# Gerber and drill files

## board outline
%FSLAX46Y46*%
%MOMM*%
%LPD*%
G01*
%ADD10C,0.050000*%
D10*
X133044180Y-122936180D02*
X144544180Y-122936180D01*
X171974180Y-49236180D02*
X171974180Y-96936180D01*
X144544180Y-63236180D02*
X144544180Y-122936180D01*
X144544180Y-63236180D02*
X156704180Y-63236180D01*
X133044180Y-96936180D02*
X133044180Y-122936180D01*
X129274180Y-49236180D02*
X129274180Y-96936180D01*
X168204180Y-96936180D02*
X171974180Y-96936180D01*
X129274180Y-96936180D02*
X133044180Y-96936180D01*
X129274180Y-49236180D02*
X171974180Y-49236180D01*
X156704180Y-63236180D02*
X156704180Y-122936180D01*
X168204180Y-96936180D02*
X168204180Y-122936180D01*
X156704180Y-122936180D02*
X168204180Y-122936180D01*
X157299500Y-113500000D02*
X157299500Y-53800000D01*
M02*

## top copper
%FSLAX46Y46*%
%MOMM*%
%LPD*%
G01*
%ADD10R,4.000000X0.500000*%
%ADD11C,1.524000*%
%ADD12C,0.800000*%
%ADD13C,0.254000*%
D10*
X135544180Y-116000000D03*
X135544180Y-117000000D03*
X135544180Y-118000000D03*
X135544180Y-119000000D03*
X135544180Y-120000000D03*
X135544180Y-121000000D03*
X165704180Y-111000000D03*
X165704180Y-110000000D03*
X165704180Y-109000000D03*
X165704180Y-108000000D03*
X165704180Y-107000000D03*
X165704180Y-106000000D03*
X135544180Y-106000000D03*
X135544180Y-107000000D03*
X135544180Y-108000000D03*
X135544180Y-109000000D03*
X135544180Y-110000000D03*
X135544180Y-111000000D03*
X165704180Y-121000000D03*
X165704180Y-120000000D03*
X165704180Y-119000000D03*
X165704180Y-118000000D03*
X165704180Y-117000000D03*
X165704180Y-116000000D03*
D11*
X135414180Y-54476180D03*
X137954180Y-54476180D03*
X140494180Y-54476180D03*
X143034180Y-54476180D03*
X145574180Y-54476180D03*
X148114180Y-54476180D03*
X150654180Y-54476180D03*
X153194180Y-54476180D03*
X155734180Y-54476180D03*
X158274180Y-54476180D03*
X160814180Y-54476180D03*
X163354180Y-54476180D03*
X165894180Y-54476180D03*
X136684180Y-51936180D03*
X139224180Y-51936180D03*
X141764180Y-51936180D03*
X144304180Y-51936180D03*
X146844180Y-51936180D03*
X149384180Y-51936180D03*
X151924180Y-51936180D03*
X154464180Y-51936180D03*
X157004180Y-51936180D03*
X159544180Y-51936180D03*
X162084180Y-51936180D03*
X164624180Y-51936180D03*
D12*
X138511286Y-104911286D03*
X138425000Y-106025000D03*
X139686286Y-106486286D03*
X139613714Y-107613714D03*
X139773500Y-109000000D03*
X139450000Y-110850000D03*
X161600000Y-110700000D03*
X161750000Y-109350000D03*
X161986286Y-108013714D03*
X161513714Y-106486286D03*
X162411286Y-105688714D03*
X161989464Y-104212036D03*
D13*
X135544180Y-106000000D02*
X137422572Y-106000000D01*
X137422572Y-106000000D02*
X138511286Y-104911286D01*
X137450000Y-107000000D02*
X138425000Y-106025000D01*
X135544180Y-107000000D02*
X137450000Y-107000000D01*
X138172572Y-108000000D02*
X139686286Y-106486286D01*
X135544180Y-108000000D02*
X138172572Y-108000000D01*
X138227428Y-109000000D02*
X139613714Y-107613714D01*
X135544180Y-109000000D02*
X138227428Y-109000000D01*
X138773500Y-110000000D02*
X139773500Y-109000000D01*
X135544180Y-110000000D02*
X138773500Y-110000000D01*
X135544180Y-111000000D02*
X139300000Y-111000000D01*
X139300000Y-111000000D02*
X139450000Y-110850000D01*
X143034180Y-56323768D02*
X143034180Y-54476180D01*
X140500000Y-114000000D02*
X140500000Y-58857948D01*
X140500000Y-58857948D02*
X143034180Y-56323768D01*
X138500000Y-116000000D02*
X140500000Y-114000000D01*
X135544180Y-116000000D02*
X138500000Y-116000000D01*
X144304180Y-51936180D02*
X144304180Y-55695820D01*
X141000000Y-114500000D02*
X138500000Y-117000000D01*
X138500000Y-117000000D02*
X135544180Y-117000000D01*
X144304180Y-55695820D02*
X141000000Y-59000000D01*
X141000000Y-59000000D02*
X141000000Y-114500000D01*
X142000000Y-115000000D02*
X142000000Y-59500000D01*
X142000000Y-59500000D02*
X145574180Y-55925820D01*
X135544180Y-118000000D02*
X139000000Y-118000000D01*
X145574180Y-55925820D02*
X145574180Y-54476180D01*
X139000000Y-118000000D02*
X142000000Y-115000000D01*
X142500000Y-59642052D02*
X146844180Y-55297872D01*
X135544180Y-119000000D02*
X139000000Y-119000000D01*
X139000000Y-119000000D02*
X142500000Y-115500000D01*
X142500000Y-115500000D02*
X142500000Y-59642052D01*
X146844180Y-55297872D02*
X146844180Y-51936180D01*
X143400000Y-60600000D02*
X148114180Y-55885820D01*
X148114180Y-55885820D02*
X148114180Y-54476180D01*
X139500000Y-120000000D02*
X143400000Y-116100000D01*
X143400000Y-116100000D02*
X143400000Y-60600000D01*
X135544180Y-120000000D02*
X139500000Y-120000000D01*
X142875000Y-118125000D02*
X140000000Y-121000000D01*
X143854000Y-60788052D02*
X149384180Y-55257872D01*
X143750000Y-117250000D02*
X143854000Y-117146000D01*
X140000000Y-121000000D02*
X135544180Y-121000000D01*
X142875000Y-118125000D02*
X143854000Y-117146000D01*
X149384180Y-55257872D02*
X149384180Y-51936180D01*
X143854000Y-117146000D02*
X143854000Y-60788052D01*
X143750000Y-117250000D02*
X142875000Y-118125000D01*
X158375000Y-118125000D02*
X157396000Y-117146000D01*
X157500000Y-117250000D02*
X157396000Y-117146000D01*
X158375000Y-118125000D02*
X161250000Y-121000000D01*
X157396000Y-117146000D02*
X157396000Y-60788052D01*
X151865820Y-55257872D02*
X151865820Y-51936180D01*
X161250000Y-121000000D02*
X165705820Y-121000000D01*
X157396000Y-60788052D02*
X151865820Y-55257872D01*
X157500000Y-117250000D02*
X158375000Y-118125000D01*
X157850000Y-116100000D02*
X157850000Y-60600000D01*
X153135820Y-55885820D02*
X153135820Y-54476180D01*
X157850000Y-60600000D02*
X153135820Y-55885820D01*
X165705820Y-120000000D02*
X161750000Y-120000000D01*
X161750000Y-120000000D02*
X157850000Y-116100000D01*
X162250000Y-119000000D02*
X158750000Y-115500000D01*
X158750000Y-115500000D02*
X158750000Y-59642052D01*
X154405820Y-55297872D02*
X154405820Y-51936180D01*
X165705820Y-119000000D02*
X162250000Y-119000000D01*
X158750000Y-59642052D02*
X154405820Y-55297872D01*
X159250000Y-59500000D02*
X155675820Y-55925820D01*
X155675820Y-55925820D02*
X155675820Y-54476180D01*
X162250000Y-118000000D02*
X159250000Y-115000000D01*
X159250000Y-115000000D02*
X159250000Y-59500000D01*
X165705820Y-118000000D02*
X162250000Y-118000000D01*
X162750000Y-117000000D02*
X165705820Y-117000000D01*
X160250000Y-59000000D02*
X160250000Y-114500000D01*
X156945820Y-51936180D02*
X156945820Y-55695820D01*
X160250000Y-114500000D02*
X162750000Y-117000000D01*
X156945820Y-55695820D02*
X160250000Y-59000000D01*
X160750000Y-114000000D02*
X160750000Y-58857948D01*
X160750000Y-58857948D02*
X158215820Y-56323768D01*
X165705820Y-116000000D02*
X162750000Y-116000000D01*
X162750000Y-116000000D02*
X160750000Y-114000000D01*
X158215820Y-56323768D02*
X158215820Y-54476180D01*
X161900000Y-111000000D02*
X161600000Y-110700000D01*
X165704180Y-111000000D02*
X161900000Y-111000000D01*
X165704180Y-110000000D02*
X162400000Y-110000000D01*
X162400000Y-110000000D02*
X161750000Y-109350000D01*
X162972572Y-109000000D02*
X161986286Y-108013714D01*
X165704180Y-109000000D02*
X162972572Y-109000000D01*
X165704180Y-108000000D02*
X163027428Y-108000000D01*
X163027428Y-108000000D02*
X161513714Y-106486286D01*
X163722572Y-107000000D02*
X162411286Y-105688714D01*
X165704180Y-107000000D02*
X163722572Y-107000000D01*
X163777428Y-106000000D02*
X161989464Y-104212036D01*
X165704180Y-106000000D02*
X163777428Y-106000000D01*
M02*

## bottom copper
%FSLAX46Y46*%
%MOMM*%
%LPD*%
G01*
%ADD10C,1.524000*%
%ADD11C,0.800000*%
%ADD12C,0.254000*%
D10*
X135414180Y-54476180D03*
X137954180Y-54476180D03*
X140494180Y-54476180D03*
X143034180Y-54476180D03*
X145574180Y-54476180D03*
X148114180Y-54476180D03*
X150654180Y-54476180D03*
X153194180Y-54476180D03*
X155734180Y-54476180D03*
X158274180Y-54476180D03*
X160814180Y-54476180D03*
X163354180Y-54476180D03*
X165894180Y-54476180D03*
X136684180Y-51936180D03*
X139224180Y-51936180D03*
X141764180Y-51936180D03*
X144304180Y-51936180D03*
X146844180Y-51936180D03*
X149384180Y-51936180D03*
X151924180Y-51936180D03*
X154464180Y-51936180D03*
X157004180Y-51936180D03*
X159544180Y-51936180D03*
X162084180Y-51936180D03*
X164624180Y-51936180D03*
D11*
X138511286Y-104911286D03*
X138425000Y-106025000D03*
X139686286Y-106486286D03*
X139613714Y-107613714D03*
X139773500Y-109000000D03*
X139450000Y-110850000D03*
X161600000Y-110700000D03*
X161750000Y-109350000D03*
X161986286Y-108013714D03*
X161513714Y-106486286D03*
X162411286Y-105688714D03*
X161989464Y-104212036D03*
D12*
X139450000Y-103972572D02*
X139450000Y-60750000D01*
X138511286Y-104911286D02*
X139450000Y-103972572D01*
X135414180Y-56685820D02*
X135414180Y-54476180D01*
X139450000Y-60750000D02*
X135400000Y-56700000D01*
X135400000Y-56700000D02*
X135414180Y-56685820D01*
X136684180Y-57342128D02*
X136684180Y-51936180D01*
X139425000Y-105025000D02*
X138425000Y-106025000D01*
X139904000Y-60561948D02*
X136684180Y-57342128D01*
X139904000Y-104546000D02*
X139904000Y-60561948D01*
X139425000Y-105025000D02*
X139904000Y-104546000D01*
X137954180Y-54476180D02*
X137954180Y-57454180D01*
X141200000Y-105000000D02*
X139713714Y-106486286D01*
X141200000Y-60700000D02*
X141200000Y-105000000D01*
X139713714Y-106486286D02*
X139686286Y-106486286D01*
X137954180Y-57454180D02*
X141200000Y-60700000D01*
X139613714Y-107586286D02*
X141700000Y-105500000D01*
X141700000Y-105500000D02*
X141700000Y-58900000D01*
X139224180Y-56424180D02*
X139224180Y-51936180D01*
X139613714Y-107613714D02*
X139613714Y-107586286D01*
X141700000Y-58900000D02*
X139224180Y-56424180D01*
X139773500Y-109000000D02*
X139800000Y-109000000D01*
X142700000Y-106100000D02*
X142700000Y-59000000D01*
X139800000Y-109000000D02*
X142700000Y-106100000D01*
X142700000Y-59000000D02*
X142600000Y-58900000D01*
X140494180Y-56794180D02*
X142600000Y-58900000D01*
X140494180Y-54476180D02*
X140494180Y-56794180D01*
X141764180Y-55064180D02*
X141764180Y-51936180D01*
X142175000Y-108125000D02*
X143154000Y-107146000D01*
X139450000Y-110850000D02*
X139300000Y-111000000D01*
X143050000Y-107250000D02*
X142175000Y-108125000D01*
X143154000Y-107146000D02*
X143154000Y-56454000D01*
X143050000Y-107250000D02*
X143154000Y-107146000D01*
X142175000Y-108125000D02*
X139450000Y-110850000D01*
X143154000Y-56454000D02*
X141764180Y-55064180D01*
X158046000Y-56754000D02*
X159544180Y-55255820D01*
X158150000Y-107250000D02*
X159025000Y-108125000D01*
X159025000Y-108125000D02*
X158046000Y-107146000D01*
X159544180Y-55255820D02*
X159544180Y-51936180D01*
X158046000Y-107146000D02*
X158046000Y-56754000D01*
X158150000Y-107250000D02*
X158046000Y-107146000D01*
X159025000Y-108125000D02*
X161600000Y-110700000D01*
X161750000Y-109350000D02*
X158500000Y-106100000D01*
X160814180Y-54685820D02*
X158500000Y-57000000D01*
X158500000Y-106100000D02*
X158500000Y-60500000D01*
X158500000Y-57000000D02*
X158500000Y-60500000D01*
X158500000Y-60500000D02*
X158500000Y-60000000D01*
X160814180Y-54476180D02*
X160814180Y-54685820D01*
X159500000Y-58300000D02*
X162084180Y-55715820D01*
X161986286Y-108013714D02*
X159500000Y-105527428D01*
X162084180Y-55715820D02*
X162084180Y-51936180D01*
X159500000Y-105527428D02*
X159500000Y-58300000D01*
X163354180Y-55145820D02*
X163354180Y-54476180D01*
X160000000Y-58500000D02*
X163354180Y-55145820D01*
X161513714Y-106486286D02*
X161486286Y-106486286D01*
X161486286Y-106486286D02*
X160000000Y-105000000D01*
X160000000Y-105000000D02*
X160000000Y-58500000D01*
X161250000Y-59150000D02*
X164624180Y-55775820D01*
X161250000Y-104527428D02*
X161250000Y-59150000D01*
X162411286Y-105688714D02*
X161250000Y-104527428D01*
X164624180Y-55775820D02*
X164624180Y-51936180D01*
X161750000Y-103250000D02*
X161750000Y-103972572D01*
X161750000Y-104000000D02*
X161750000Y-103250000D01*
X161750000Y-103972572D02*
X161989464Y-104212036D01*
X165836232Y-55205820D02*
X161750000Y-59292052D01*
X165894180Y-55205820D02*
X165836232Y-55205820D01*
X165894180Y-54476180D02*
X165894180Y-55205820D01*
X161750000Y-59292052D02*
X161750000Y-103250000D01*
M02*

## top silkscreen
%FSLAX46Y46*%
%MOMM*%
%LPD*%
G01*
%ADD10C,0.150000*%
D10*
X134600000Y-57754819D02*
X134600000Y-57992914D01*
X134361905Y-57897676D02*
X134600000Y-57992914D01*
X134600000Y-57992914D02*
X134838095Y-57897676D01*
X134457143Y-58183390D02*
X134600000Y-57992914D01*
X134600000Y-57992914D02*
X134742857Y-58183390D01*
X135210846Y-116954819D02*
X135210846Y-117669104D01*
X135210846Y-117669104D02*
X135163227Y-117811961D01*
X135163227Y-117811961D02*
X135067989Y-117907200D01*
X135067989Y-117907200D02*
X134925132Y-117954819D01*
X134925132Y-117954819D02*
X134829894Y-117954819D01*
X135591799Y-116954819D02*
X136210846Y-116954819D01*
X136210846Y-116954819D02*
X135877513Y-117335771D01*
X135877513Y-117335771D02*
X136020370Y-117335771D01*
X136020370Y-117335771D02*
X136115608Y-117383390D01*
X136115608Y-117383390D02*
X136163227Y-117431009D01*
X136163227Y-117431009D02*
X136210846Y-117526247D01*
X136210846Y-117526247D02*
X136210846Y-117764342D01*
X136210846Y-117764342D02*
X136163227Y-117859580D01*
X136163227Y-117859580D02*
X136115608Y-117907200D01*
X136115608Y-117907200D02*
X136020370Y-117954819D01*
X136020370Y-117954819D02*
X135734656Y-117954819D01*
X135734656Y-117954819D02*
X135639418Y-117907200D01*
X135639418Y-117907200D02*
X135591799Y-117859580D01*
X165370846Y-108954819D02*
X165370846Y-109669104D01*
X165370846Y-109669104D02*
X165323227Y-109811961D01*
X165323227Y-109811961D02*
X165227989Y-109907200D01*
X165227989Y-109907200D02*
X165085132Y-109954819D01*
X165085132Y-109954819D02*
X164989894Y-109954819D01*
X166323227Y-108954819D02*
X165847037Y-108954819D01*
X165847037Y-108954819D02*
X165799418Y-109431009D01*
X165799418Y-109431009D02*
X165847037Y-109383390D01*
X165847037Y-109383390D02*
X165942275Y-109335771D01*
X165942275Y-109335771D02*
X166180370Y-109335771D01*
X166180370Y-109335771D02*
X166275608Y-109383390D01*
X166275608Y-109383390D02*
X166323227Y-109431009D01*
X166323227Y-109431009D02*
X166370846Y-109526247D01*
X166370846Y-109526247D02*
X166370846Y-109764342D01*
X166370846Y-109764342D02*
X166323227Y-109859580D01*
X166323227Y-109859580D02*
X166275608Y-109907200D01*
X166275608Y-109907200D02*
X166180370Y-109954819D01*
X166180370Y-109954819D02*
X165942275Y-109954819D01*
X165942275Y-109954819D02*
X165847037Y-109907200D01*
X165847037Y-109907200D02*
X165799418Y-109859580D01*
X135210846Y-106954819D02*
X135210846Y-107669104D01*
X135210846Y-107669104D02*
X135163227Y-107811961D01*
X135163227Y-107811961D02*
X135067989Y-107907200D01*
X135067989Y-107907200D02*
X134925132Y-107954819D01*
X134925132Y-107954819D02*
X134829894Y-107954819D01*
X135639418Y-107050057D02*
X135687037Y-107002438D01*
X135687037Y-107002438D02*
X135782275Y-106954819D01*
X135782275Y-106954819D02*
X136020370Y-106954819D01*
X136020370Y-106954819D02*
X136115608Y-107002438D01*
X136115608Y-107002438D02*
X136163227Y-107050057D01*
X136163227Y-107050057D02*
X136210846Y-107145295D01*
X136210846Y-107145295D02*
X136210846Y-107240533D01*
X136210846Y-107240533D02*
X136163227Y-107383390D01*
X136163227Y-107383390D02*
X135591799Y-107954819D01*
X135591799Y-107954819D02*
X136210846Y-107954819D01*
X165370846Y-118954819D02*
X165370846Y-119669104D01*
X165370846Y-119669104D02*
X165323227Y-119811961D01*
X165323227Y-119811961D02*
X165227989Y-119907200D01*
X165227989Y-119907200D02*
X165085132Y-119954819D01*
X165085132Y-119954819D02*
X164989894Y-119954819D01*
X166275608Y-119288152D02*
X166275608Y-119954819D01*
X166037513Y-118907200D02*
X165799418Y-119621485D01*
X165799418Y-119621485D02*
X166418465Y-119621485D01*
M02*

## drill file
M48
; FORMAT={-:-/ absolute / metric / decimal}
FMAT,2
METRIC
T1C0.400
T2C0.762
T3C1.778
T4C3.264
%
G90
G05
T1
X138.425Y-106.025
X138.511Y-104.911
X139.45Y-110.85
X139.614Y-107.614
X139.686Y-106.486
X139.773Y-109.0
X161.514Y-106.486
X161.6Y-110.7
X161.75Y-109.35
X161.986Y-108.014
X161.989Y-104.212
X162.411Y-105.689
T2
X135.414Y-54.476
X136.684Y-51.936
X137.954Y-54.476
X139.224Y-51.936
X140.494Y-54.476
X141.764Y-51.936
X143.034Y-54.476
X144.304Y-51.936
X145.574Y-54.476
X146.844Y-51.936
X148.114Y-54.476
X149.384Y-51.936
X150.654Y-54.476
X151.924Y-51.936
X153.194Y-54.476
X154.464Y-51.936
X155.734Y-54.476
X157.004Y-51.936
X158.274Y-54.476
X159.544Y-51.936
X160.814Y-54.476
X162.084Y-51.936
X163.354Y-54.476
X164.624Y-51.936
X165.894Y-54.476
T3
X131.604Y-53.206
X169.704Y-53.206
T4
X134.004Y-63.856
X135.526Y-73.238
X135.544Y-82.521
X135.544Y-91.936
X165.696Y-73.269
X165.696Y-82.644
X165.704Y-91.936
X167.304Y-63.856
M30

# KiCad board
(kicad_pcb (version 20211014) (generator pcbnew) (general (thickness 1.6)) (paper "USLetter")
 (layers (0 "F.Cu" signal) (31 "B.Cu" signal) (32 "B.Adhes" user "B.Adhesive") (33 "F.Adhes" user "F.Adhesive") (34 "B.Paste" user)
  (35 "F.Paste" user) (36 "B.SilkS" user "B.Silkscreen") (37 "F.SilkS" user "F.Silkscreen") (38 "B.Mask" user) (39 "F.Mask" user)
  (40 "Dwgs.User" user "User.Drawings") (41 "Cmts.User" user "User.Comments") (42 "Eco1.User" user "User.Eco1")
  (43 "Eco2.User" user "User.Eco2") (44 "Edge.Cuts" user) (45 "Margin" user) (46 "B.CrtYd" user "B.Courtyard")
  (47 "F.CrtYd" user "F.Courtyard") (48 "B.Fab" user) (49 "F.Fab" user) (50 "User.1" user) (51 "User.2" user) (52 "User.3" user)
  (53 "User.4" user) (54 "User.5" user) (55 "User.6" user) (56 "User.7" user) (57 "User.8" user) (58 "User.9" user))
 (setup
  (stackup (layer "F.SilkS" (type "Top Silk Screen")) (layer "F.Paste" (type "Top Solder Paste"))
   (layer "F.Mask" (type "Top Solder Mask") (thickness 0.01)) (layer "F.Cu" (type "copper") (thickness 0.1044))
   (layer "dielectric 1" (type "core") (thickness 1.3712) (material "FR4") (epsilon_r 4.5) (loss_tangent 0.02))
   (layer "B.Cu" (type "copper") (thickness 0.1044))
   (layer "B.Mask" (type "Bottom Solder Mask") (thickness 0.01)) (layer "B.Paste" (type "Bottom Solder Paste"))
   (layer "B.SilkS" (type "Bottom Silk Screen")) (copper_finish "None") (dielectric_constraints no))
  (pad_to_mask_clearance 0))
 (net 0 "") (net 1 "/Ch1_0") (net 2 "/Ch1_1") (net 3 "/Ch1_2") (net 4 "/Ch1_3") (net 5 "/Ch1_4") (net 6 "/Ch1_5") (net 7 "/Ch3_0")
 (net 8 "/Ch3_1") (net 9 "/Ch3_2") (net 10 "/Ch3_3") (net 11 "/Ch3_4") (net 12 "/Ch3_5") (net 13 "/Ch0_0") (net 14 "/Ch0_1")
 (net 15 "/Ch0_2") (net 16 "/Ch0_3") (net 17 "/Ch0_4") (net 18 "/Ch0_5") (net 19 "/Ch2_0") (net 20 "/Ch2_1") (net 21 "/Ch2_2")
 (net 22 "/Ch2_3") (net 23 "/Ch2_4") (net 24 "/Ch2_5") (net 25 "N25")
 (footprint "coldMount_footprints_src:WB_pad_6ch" (layer "F.Cu") (at 135.54418 118.5 -90)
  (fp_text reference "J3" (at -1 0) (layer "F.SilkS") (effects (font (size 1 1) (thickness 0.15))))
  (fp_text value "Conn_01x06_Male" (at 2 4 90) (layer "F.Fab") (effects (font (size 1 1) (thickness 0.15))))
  (pad "1" connect rect (at -2.5 0 270) (size 0.5 4) (layers "F.Cu" "F.Mask") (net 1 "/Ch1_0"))
  (pad "2" connect rect (at -1.5 0 270) (size 0.5 4) (layers "F.Cu" "F.Mask") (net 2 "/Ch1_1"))
  (pad "3" connect rect (at -0.5 0 270) (size 0.5 4) (layers "F.Cu" "F.Mask") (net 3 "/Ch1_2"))
  (pad "4" connect rect (at 0.5 0 270) (size 0.5 4) (layers "F.Cu" "F.Mask") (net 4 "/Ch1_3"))
  (pad "5" connect rect (at 1.5 0 270) (size 0.5 4) (layers "F.Cu" "F.Mask") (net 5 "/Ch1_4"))
  (pad "6" connect rect (at 2.5 0 270) (size 0.5 4) (layers "F.Cu" "F.Mask") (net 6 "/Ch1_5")))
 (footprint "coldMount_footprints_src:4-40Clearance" (layer "F.Cu") (at 135.54354 82.52076)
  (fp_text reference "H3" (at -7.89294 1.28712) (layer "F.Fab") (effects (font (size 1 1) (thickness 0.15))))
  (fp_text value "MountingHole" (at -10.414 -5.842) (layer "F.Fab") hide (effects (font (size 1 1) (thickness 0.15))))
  (pad "" np_thru_hole circle (at 0 0) (size 3.2639 3.2639) (drill 3.2639) (layers F&B.Cu *.Mask)))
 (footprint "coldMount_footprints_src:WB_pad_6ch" (layer "F.Cu") (at 165.70418 108.5 90)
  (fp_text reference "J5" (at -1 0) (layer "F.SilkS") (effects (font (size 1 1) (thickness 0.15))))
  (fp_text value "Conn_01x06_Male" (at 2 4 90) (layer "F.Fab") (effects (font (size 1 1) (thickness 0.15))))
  (pad "1" connect rect (at -2.5 0 90) (size 0.5 4) (layers "F.Cu" "F.Mask") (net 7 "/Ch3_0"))
  (pad "2" connect rect (at -1.5 0 90) (size 0.5 4) (layers "F.Cu" "F.Mask") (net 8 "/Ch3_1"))
  (pad "3" connect rect (at -0.5 0 90) (size 0.5 4) (layers "F.Cu" "F.Mask") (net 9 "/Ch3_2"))
  (pad "4" connect rect (at 0.5 0 90) (size 0.5 4) (layers "F.Cu" "F.Mask") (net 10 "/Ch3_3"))
  (pad "5" connect rect (at 1.5 0 90) (size 0.5 4) (layers "F.Cu" "F.Mask") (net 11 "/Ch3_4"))
  (pad "6" connect rect (at 2.5 0 90) (size 0.5 4) (layers "F.Cu" "F.Mask") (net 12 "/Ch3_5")))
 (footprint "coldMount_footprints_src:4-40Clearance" (layer "F.Cu") (at 165.69586 73.26852)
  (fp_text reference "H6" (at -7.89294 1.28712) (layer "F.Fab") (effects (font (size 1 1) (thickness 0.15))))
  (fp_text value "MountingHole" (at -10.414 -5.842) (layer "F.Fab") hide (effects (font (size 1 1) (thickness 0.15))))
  (pad "" np_thru_hole circle (at 0 0) (size 3.2639 3.2639) (drill 3.2639) (layers F&B.Cu *.Mask)))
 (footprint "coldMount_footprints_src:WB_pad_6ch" (layer "F.Cu") (at 135.54418 108.5 -90)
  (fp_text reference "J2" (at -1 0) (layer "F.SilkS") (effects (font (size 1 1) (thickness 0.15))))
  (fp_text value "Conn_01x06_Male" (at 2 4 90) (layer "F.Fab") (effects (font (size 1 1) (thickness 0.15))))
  (pad "1" connect rect (at -2.5 0 270) (size 0.5 4) (layers "F.Cu" "F.Mask") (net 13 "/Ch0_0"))
  (pad "2" connect rect (at -1.5 0 270) (size 0.5 4) (layers "F.Cu" "F.Mask") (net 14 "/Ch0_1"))
  (pad "3" connect rect (at -0.5 0 270) (size 0.5 4) (layers "F.Cu" "F.Mask") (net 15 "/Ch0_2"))
  (pad "4" connect rect (at 0.5 0 270) (size 0.5 4) (layers "F.Cu" "F.Mask") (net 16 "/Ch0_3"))
  (pad "5" connect rect (at 1.5 0 270) (size 0.5 4) (layers "F.Cu" "F.Mask") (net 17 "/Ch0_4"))
  (pad "6" connect rect (at 2.5 0 270) (size 0.5 4) (layers "F.Cu" "F.Mask") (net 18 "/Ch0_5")))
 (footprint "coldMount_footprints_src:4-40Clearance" (layer "F.Cu") (at 167.30418 63.85618)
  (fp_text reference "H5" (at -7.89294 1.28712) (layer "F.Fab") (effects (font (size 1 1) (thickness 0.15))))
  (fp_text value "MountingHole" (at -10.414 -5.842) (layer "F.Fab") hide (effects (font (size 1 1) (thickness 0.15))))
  (pad "" np_thru_hole circle (at 0 0) (size 3.2639 3.2639) (drill 3.2639) (layers F&B.Cu *.Mask)))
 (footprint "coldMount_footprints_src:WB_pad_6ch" (layer "F.Cu") (at 165.70418 118.5 90)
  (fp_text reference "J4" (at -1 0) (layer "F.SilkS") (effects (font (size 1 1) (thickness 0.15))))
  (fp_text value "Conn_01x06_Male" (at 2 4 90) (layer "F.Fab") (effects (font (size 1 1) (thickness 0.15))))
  (pad "1" connect rect (at -2.5 0 90) (size 0.5 4) (layers "F.Cu" "F.Mask") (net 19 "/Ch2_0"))
  (pad "2" connect rect (at -1.5 0 90) (size 0.5 4) (layers "F.Cu" "F.Mask") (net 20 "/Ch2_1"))
  (pad "3" connect rect (at -0.5 0 90) (size 0.5 4) (layers "F.Cu" "F.Mask") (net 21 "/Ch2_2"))
  (pad "4" connect rect (at 0.5 0 90) (size 0.5 4) (layers "F.Cu" "F.Mask") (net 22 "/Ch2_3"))
  (pad "5" connect rect (at 1.5 0 90) (size 0.5 4) (layers "F.Cu" "F.Mask") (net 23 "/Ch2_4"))
  (pad "6" connect rect (at 2.5 0 90) (size 0.5 4) (layers "F.Cu" "F.Mask") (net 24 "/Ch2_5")))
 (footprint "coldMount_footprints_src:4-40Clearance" (layer "F.Cu") (at 165.69586 82.6439)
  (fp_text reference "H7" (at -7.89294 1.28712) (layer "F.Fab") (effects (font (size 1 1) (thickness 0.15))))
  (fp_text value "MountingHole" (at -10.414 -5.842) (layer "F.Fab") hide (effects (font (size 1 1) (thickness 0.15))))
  (pad "" np_thru_hole circle (at 0 0) (size 3.2639 3.2639) (drill 3.2639) (layers F&B.Cu *.Mask)))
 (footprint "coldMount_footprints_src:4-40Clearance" (layer "F.Cu") (at 135.52576 73.23828)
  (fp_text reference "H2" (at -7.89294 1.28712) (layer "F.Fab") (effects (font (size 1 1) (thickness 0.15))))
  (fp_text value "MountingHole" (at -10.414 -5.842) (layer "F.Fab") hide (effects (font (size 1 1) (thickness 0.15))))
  (pad "" np_thru_hole circle (at 0 0) (size 3.2639 3.2639) (drill 3.2639) (layers F&B.Cu *.Mask)))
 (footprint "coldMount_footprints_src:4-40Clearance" (layer "F.Cu") (at 135.54418 91.93618)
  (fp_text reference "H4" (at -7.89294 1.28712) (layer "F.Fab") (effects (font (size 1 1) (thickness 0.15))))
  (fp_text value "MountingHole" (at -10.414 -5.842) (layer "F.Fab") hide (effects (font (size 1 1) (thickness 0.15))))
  (pad "" np_thru_hole circle (at 0 0) (size 3.2639 3.2639) (drill 3.2639) (layers F&B.Cu *.Mask)))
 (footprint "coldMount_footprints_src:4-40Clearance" (layer "F.Cu") (at 165.70418 91.93618)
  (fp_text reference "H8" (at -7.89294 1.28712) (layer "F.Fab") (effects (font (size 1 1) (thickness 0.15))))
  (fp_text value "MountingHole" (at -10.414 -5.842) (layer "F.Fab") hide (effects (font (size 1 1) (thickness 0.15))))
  (pad "" np_thru_hole circle (at 0 0) (size 3.2639 3.2639) (drill 3.2639) (layers F&B.Cu *.Mask)))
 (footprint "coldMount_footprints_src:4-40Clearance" (layer "F.Cu") (at 134.00418 63.85618)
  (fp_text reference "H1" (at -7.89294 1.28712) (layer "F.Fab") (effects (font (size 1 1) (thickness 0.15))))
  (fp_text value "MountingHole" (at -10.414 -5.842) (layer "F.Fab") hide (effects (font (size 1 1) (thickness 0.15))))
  (pad "" np_thru_hole circle (at 0 0) (size 3.2639 3.2639) (drill 3.2639) (layers F&B.Cu *.Mask)))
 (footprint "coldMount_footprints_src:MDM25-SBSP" (layer "B.Cu") (at 150.65418 54.47618 180)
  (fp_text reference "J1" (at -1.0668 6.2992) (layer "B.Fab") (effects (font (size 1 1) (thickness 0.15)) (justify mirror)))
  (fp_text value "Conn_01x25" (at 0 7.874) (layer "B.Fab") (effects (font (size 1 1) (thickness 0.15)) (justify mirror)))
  (pad "" np_thru_hole circle (at 19.05 1.27 180) (size 1.778 1.778) (drill 1.778) (layers F&B.Cu *.Mask))
  (pad "" np_thru_hole circle (at -19.05 1.27 180) (size 1.778 1.778) (drill 1.778) (layers F&B.Cu *.Mask))
  (pad "1" thru_hole circle (at 15.24 0 180) (size 1.524 1.524) (drill 0.762) (layers F&B.Cu *.Mask) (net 13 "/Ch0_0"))
  (pad "2" thru_hole circle (at 12.7 0 180) (size 1.524 1.524) (drill 0.762) (layers F&B.Cu *.Mask) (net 15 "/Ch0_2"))
  (pad "3" thru_hole circle (at 10.16 0 180) (size 1.524 1.524) (drill 0.762) (layers F&B.Cu *.Mask) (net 17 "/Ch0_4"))
  (pad "4" thru_hole circle (at 7.62 0 180) (size 1.524 1.524) (drill 0.762) (layers F&B.Cu *.Mask) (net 1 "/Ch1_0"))
  (pad "5" thru_hole circle (at 5.08 0 180) (size 1.524 1.524) (drill 0.762) (layers F&B.Cu *.Mask) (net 3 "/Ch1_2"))
  (pad "6" thru_hole circle (at 2.54 0 180) (size 1.524 1.524) (drill 0.762) (layers F&B.Cu *.Mask) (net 5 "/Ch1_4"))
  (pad "7" thru_hole circle (at 0 0 180) (size 1.524 1.524) (drill 0.762) (layers F&B.Cu *.Mask) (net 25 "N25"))
  (pad "8" thru_hole circle (at -2.54 0 180) (size 1.524 1.524) (drill 0.762) (layers F&B.Cu *.Mask) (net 20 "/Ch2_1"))
  (pad "9" thru_hole circle (at -5.08 0 180) (size 1.524 1.524) (drill 0.762) (layers F&B.Cu *.Mask) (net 22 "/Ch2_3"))
  (pad "10" thru_hole circle (at -7.62 0 180) (size 1.524 1.524) (drill 0.762) (layers F&B.Cu *.Mask) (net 24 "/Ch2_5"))
  (pad "11" thru_hole circle (at -10.16 0 180) (size 1.524 1.524) (drill 0.762) (layers F&B.Cu *.Mask) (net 8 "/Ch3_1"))
  (pad "12" thru_hole circle (at -12.7 0 180) (size 1.524 1.524) (drill 0.762) (layers F&B.Cu *.Mask) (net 10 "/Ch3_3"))
  (pad "13" thru_hole circle (at -15.24 0 180) (size 1.524 1.524) (drill 0.762) (layers F&B.Cu *.Mask) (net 12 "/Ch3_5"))
  (pad "14" thru_hole circle (at 13.97 2.54 180) (size 1.524 1.524) (drill 0.762) (layers F&B.Cu *.Mask) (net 14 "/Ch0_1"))
  (pad "15" thru_hole circle (at 11.43 2.54 180) (size 1.524 1.524) (drill 0.762) (layers F&B.Cu *.Mask) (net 16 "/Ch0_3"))
  (pad "16" thru_hole circle (at 8.89 2.54 180) (size 1.524 1.524) (drill 0.762) (layers F&B.Cu *.Mask) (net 18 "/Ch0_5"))
  (pad "17" thru_hole circle (at 6.35 2.54 180) (size 1.524 1.524) (drill 0.762) (layers F&B.Cu *.Mask) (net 2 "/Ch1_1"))
  (pad "18" thru_hole circle (at 3.81 2.54 180) (size 1.524 1.524) (drill 0.762) (layers F&B.Cu *.Mask) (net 4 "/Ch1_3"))
  (pad "19" thru_hole circle (at 1.27 2.54 180) (size 1.524 1.524) (drill 0.762) (layers F&B.Cu *.Mask) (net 6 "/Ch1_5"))
  (pad "20" thru_hole circle (at -1.27 2.54 180) (size 1.524 1.524) (drill 0.762) (layers F&B.Cu *.Mask) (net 19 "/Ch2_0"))
  (pad "21" thru_hole circle (at -3.81 2.54 180) (size 1.524 1.524) (drill 0.762) (layers F&B.Cu *.Mask) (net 21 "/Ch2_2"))
  (pad "22" thru_hole circle (at -6.35 2.54 180) (size 1.524 1.524) (drill 0.762) (layers F&B.Cu *.Mask) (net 23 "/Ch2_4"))
  (pad "23" thru_hole circle (at -8.89 2.54 180) (size 1.524 1.524) (drill 0.762) (layers F&B.Cu *.Mask) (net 7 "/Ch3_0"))
  (pad "24" thru_hole circle (at -11.43 2.54 180) (size 1.524 1.524) (drill 0.762) (layers F&B.Cu *.Mask) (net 9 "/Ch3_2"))
  (pad "25" thru_hole circle (at -13.97 2.54 180) (size 1.524 1.524) (drill 0.762) (layers F&B.Cu *.Mask) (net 11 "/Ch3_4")))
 (gr_line (start 133.04418 122.93618) (end 144.54418 122.93618) (layer "Edge.Cuts") (width 0.05))
 (gr_line (start 171.97418 49.23618) (end 171.97418 96.93618) (layer "Edge.Cuts") (width 0.05))
 (gr_line (start 144.54418 63.23618) (end 144.54418 122.93618) (layer "Edge.Cuts") (width 0.05))
 (gr_line (start 144.54418 63.23618) (end 156.70418 63.23618) (layer "Edge.Cuts") (width 0.05))
 (gr_line (start 133.04418 96.93618) (end 133.04418 122.93618) (layer "Edge.Cuts") (width 0.05))
 (gr_line (start 129.27418 49.23618) (end 129.27418 96.93618) (layer "Edge.Cuts") (width 0.05))
 (gr_line (start 168.20418 96.93618) (end 171.97418 96.93618) (layer "Edge.Cuts") (width 0.05))
 (gr_line (start 129.27418 96.93618) (end 133.04418 96.93618) (layer "Edge.Cuts") (width 0.05))
 (gr_line (start 129.27418 49.23618) (end 171.97418 49.23618) (layer "Edge.Cuts") (width 0.05))
 (gr_line (start 156.70418 63.23618) (end 156.70418 122.93618) (layer "Edge.Cuts") (width 0.05))
 (gr_line (start 168.20418 96.93618) (end 168.20418 122.93618) (layer "Edge.Cuts") (width 0.05))
 (gr_line (start 156.70418 122.93618) (end 168.20418 122.93618) (layer "Edge.Cuts") (width 0.05))
 (gr_line (start 157.2995 113.5) (end 157.2995 53.8) (layer "Edge.Cuts") (width 0.05))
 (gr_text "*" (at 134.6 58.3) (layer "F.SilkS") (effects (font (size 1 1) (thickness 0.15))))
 (segment (start 135.54418 106) (end 137.422572 106) (width 0.254) (layer "F.Cu") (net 13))
 (segment (start 137.422572 106) (end 138.511286 104.911286) (width 0.254) (layer "F.Cu") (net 13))
 (via (at 138.511286 104.911286) (size 0.8) (drill 0.4) (layers "F.Cu" "B.Cu") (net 13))
 (segment (start 139.45 103.972572) (end 139.45 60.75) (width 0.254) (layer "B.Cu") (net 13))
 (segment (start 138.511286 104.911286) (end 139.45 103.972572) (width 0.254) (layer "B.Cu") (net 13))
 (segment (start 135.41418 56.68582) (end 135.41418 54.47618) (width 0.254) (layer "B.Cu") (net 13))
 (segment (start 139.45 60.75) (end 135.4 56.7) (width 0.254) (layer "B.Cu") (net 13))
 (segment (start 135.4 56.7) (end 135.41418 56.68582) (width 0.254) (layer "B.Cu") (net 13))
 (segment (start 137.45 107) (end 138.425 106.025) (width 0.254) (layer "F.Cu") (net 14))
 (segment (start 135.54418 107) (end 137.45 107) (width 0.254) (layer "F.Cu") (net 14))
 (via (at 138.425 106.025) (size 0.8) (drill 0.4) (layers "F.Cu" "B.Cu") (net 14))
 (segment (start 136.68418 57.342128) (end 136.68418 51.93618) (width 0.254) (layer "B.Cu") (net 14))
 (segment (start 139.425 105.025) (end 138.425 106.025) (width 0.254) (layer "B.Cu") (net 14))
 (segment (start 139.904 60.561948) (end 136.68418 57.342128) (width 0.254) (layer "B.Cu") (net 14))
 (segment (start 139.904 104.546) (end 139.904 60.561948) (width 0.254) (layer "B.Cu") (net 14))
 (segment (start 139.425 105.025) (end 139.904 104.546) (width 0.254) (layer "B.Cu") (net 14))
 (segment (start 138.172572 108) (end 139.686286 106.486286) (width 0.254) (layer "F.Cu") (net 15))
 (segment (start 135.54418 108) (end 138.172572 108) (width 0.254) (layer "F.Cu") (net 15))
 (via (at 139.686286 106.486286) (size 0.8) (drill 0.4) (layers "F.Cu" "B.Cu") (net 15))
 (segment (start 137.95418 54.47618) (end 137.95418 57.45418) (width 0.254) (layer "B.Cu") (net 15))
 (segment (start 141.2 105) (end 139.713714 106.486286) (width 0.254) (layer "B.Cu") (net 15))
 (segment (start 141.2 60.7) (end 141.2 105) (width 0.254) (layer "B.Cu") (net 15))
 (segment (start 139.713714 106.486286) (end 139.686286 106.486286) (width 0.254) (layer "B.Cu") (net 15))
 (segment (start 137.95418 57.45418) (end 141.2 60.7) (width 0.254) (layer "B.Cu") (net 15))
 (segment (start 138.227428 109) (end 139.613714 107.613714) (width 0.254) (layer "F.Cu") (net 16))
 (segment (start 135.54418 109) (end 138.227428 109) (width 0.254) (layer "F.Cu") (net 16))
 (via (at 139.613714 107.613714) (size 0.8) (drill 0.4) (layers "F.Cu" "B.Cu") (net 16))
 (segment (start 139.613714 107.586286) (end 141.7 105.5) (width 0.254) (layer "B.Cu") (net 16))
 (segment (start 141.7 105.5) (end 141.7 58.9) (width 0.254) (layer "B.Cu") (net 16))
 (segment (start 139.22418 56.42418) (end 139.22418 51.93618) (width 0.254) (layer "B.Cu") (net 16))
 (segment (start 139.613714 107.613714) (end 139.613714 107.586286) (width 0.254) (layer "B.Cu") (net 16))
 (segment (start 141.7 58.9) (end 139.22418 56.42418) (width 0.254) (layer "B.Cu") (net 16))
 (segment (start 138.7735 110) (end 139.7735 109) (width 0.254) (layer "F.Cu") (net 17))
 (segment (start 135.54418 110) (end 138.7735 110) (width 0.254) (layer "F.Cu") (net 17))
 (via (at 139.7735 109) (size 0.8) (drill 0.4) (layers "F.Cu" "B.Cu") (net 17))
 (segment (start 139.7735 109) (end 139.8 109) (width 0.254) (layer "B.Cu") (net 17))
 (segment (start 142.7 106.1) (end 142.7 59) (width 0.254) (layer "B.Cu") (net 17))
 (segment (start 139.8 109) (end 142.7 106.1) (width 0.254) (layer "B.Cu") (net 17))
 (segment (start 142.7 59) (end 142.6 58.9) (width 0.254) (layer "B.Cu") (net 17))
 (segment (start 140.49418 56.79418) (end 142.6 58.9) (width 0.254) (layer "B.Cu") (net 17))
 (segment (start 140.49418 54.47618) (end 140.49418 56.79418) (width 0.254) (layer "B.Cu") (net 17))
 (segment (start 135.54418 111) (end 139.3 111) (width 0.254) (layer "F.Cu") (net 18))
 (segment (start 139.3 111) (end 139.45 110.85) (width 0.254) (layer "F.Cu") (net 18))
 (via (at 139.45 110.85) (size 0.8) (drill 0.4) (layers "F.Cu" "B.Cu") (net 18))
 (segment (start 141.76418 55.06418) (end 141.76418 51.93618) (width 0.254) (layer "B.Cu") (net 18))
 (segment (start 142.175 108.125) (end 143.154 107.146) (width 0.254) (layer "B.Cu") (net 18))
 (segment (start 139.45 110.85) (end 139.3 111) (width 0.254) (layer "B.Cu") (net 18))
 (segment (start 143.05 107.25) (end 142.175 108.125) (width 0.254) (layer "B.Cu") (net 18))
 (segment (start 143.154 107.146) (end 143.154 56.454) (width 0.254) (layer "B.Cu") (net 18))
 (segment (start 143.05 107.25) (end 143.154 107.146) (width 0.254) (layer "B.Cu") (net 18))
 (segment (start 142.175 108.125) (end 139.45 110.85) (width 0.254) (layer "B.Cu") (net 18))
 (segment (start 143.154 56.454) (end 141.76418 55.06418) (width 0.254) (layer "B.Cu") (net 18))
 (segment (start 143.03418 56.323768) (end 143.03418 54.47618) (width 0.254) (layer "F.Cu") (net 1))
 (segment (start 140.5 114) (end 140.5 58.857948) (width 0.254) (layer "F.Cu") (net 1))
 (segment (start 140.5 58.857948) (end 143.03418 56.323768) (width 0.254) (layer "F.Cu") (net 1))
 (segment (start 138.5 116) (end 140.5 114) (width 0.254) (layer "F.Cu") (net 1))
 (segment (start 135.54418 116) (end 138.5 116) (width 0.254) (layer "F.Cu") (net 1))
 (segment (start 144.30418 51.93618) (end 144.30418 55.69582) (width 0.254) (layer "F.Cu") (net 2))
 (segment (start 141 114.5) (end 138.5 117) (width 0.254) (layer "F.Cu") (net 2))
 (segment (start 138.5 117) (end 135.54418 117) (width 0.254) (layer "F.Cu") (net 2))
 (segment (start 144.30418 55.69582) (end 141 59) (width 0.254) (layer "F.Cu") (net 2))
 (segment (start 141 59) (end 141 114.5) (width 0.254) (layer "F.Cu") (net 2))
 (segment (start 142 115) (end 142 59.5) (width 0.254) (layer "F.Cu") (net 3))
 (segment (start 142 59.5) (end 145.57418 55.92582) (width 0.254) (layer "F.Cu") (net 3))
 (segment (start 135.54418 118) (end 139 118) (width 0.254) (layer "F.Cu") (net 3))
 (segment (start 145.57418 55.92582) (end 145.57418 54.47618) (width 0.254) (layer "F.Cu") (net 3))
 (segment (start 139 118) (end 142 115) (width 0.254) (layer "F.Cu") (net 3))
 (segment (start 142.5 59.642052) (end 146.84418 55.297872) (width 0.254) (layer "F.Cu") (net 4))
 (segment (start 135.54418 119) (end 139 119) (width 0.254) (layer "F.Cu") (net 4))
 (segment (start 139 119) (end 142.5 115.5) (width 0.254) (layer "F.Cu") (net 4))
 (segment (start 142.5 115.5) (end 142.5 59.642052) (width 0.254) (layer "F.Cu") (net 4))
 (segment (start 146.84418 55.297872) (end 146.84418 51.93618) (width 0.254) (layer "F.Cu") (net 4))
 (segment (start 143.4 60.6) (end 148.11418 55.88582) (width 0.254) (layer "F.Cu") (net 5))
 (segment (start 148.11418 55.88582) (end 148.11418 54.47618) (width 0.254) (layer "F.Cu") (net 5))
 (segment (start 139.5 120) (end 143.4 116.1) (width 0.254) (layer "F.Cu") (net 5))
 (segment (start 143.4 116.1) (end 143.4 60.6) (width 0.254) (layer "F.Cu") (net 5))
 (segment (start 135.54418 120) (end 139.5 120) (width 0.254) (layer "F.Cu") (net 5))
 (segment (start 142.875 118.125) (end 140 121) (width 0.254) (layer "F.Cu") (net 6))
 (segment (start 143.854 60.788052) (end 149.38418 55.257872) (width 0.254) (layer "F.Cu") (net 6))
 (segment (start 143.75 117.25) (end 143.854 117.146) (width 0.254) (layer "F.Cu") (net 6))
 (segment (start 140 121) (end 135.54418 121) (width 0.254) (layer "F.Cu") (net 6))
 (segment (start 142.875 118.125) (end 143.854 117.146) (width 0.254) (layer "F.Cu") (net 6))
 (segment (start 149.38418 55.257872) (end 149.38418 51.93618) (width 0.254) (layer "F.Cu") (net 6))
 (segment (start 143.854 117.146) (end 143.854 60.788052) (width 0.254) (layer "F.Cu") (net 6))
 (segment (start 143.75 117.25) (end 142.875 118.125) (width 0.254) (layer "F.Cu") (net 6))
 (segment (start 158.375 118.125) (end 157.396 117.146) (width 0.254) (layer "F.Cu") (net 19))
 (segment (start 157.5 117.25) (end 157.396 117.146) (width 0.254) (layer "F.Cu") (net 19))
 (segment (start 158.375 118.125) (end 161.25 121) (width 0.254) (layer "F.Cu") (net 19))
 (segment (start 157.396 117.146) (end 157.396 60.788052) (width 0.254) (layer "F.Cu") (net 19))
 (segment (start 151.86582 55.257872) (end 151.86582 51.93618) (width 0.254) (layer "F.Cu") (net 19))
 (segment (start 161.25 121) (end 165.70582 121) (width 0.254) (layer "F.Cu") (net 19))
 (segment (start 157.396 60.788052) (end 151.86582 55.257872) (width 0.254) (layer "F.Cu") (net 19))
 (segment (start 157.5 117.25) (end 158.375 118.125) (width 0.254) (layer "F.Cu") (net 19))
 (segment (start 157.85 116.1) (end 157.85 60.6) (width 0.254) (layer "F.Cu") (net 20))
 (segment (start 153.13582 55.88582) (end 153.13582 54.47618) (width 0.254) (layer "F.Cu") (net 20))
 (segment (start 157.85 60.6) (end 153.13582 55.88582) (width 0.254) (layer "F.Cu") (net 20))
 (segment (start 165.70582 120) (end 161.75 120) (width 0.254) (layer "F.Cu") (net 20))
 (segment (start 161.75 120) (end 157.85 116.1) (width 0.254) (layer "F.Cu") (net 20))
 (segment (start 162.25 119) (end 158.75 115.5) (width 0.254) (layer "F.Cu") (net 21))
 (segment (start 158.75 115.5) (end 158.75 59.642052) (width 0.254) (layer "F.Cu") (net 21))
 (segment (start 154.40582 55.297872) (end 154.40582 51.93618) (width 0.254) (layer "F.Cu") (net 21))
 (segment (start 165.70582 119) (end 162.25 119) (width 0.254) (layer "F.Cu") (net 21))
 (segment (start 158.75 59.642052) (end 154.40582 55.297872) (width 0.254) (layer "F.Cu") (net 21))
 (segment (start 159.25 59.5) (end 155.67582 55.92582) (width 0.254) (layer "F.Cu") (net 22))
 (segment (start 155.67582 55.92582) (end 155.67582 54.47618) (width 0.254) (layer "F.Cu") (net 22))
 (segment (start 162.25 118) (end 159.25 115) (width 0.254) (layer "F.Cu") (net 22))
 (segment (start 159.25 115) (end 159.25 59.5) (width 0.254) (layer "F.Cu") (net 22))
 (segment (start 165.70582 118) (end 162.25 118) (width 0.254) (layer "F.Cu") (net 22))
 (segment (start 162.75 117) (end 165.70582 117) (width 0.254) (layer "F.Cu") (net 23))
 (segment (start 160.25 59) (end 160.25 114.5) (width 0.254) (layer "F.Cu") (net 23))
 (segment (start 156.94582 51.93618) (end 156.94582 55.69582) (width 0.254) (layer "F.Cu") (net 23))
 (segment (start 160.25 114.5) (end 162.75 117) (width 0.254) (layer "F.Cu") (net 23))
 (segment (start 156.94582 55.69582) (end 160.25 59) (width 0.254) (layer "F.Cu") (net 23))
 (segment (start 160.75 114) (end 160.75 58.857948) (width 0.254) (layer "F.Cu") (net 24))
 (segment (start 160.75 58.857948) (end 158.21582 56.323768) (width 0.254) (layer "F.Cu") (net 24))
 (segment (start 165.70582 116) (end 162.75 116) (width 0.254) (layer "F.Cu") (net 24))
 (segment (start 162.75 116) (end 160.75 114) (width 0.254) (layer "F.Cu") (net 24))
 (segment (start 158.21582 56.323768) (end 158.21582 54.47618) (width 0.254) (layer "F.Cu") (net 24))
 (segment (start 161.9 111) (end 161.6 110.7) (width 0.254) (layer "F.Cu") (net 7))
 (segment (start 165.70418 111) (end 161.9 111) (width 0.254) (layer "F.Cu") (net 7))
 (via (at 161.6 110.7) (size 0.8) (drill 0.4) (layers "F.Cu" "B.Cu") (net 7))
 (segment (start 158.046 56.754) (end 159.54418 55.25582) (width 0.254) (layer "B.Cu") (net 7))
 (segment (start 158.15 107.25) (end 159.025 108.125) (width 0.254) (layer "B.Cu") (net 7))
 (segment (start 159.025 108.125) (end 158.046 107.146) (width 0.254) (layer "B.Cu") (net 7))
 (segment (start 159.54418 55.25582) (end 159.54418 51.93618) (width 0.254) (layer "B.Cu") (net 7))
 (segment (start 158.046 107.146) (end 158.046 56.754) (width 0.254) (layer "B.Cu") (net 7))
 (segment (start 158.15 107.25) (end 158.046 107.146) (width 0.254) (layer "B.Cu") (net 7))
 (segment (start 159.025 108.125) (end 161.6 110.7) (width 0.254) (layer "B.Cu") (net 7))
 (segment (start 165.70418 110) (end 162.4 110) (width 0.254) (layer "F.Cu") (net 8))
 (segment (start 162.4 110) (end 161.75 109.35) (width 0.254) (layer "F.Cu") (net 8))
 (via (at 161.75 109.35) (size 0.8) (drill 0.4) (layers "F.Cu" "B.Cu") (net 8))
 (segment (start 161.75 109.35) (end 158.5 106.1) (width 0.254) (layer "B.Cu") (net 8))
 (segment (start 160.81418 54.68582) (end 158.5 57) (width 0.254) (layer "B.Cu") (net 8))
 (segment (start 158.5 106.1) (end 158.5 60.5) (width 0.254) (layer "B.Cu") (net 8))
 (segment (start 158.5 57) (end 158.5 60.5) (width 0.254) (layer "B.Cu") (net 8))
 (segment (start 158.5 60.5) (end 158.5 60) (width 0.254) (layer "B.Cu") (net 8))
 (segment (start 160.81418 54.47618) (end 160.81418 54.68582) (width 0.254) (layer "B.Cu") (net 8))
 (segment (start 162.972572 109) (end 161.986286 108.013714) (width 0.254) (layer "F.Cu") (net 9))
 (segment (start 165.70418 109) (end 162.972572 109) (width 0.254) (layer "F.Cu") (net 9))
 (via (at 161.986286 108.013714) (size 0.8) (drill 0.4) (layers "F.Cu" "B.Cu") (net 9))
 (segment (start 159.5 58.3) (end 162.08418 55.71582) (width 0.254) (layer "B.Cu") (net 9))
 (segment (start 161.986286 108.013714) (end 159.5 105.527428) (width 0.254) (layer "B.Cu") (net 9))
 (segment (start 162.08418 55.71582) (end 162.08418 51.93618) (width 0.254) (layer "B.Cu") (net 9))
 (segment (start 159.5 105.527428) (end 159.5 58.3) (width 0.254) (layer "B.Cu") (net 9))
 (segment (start 165.70418 108) (end 163.027428 108) (width 0.254) (layer "F.Cu") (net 10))
 (segment (start 163.027428 108) (end 161.513714 106.486286) (width 0.254) (layer "F.Cu") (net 10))
 (via (at 161.513714 106.486286) (size 0.8) (drill 0.4) (layers "F.Cu" "B.Cu") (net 10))
 (segment (start 163.35418 55.14582) (end 163.35418 54.47618) (width 0.254) (layer "B.Cu") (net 10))
 (segment (start 160 58.5) (end 163.35418 55.14582) (width 0.254) (layer "B.Cu") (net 10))
 (segment (start 161.513714 106.486286) (end 161.486286 106.486286) (width 0.254) (layer "B.Cu") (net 10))
 (segment (start 161.486286 106.486286) (end 160 105) (width 0.254) (layer "B.Cu") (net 10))
 (segment (start 160 105) (end 160 58.5) (width 0.254) (layer "B.Cu") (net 10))
 (segment (start 163.722572 107) (end 162.411286 105.688714) (width 0.254) (layer "F.Cu") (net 11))
 (segment (start 165.70418 107) (end 163.722572 107) (width 0.254) (layer "F.Cu") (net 11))
 (via (at 162.411286 105.688714) (size 0.8) (drill 0.4) (layers "F.Cu" "B.Cu") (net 11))
 (segment (start 161.25 59.15) (end 164.62418 55.77582) (width 0.254) (layer "B.Cu") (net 11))
 (segment (start 161.25 104.527428) (end 161.25 59.15) (width 0.254) (layer "B.Cu") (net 11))
 (segment (start 162.411286 105.688714) (end 161.25 104.527428) (width 0.254) (layer "B.Cu") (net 11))
 (segment (start 164.62418 55.77582) (end 164.62418 51.93618) (width 0.254) (layer "B.Cu") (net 11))
 (segment (start 163.777428 106) (end 161.989464 104.212036) (width 0.254) (layer "F.Cu") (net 12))
 (segment (start 165.70418 106) (end 163.777428 106) (width 0.254) (layer "F.Cu") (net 12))
 (via (at 161.989464 104.212036) (size 0.8) (drill 0.4) (layers "F.Cu" "B.Cu") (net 12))
 (segment (start 161.75 103.25) (end 161.75 103.972572) (width 0.254) (layer "B.Cu") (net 12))
 (segment (start 161.75 104) (end 161.75 103.25) (width 0.254) (layer "B.Cu") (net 12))
 (segment (start 161.75 103.972572) (end 161.989464 104.212036) (width 0.254) (layer "B.Cu") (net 12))
 (segment (start 165.836232 55.20582) (end 161.75 59.292052) (width 0.254) (layer "B.Cu") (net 12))
 (segment (start 165.89418 55.20582) (end 165.836232 55.20582) (width 0.254) (layer "B.Cu") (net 12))
 (segment (start 165.89418 54.47618) (end 165.89418 55.20582) (width 0.254) (layer "B.Cu") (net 12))
 (segment (start 161.75 59.292052) (end 161.75 103.25) (width 0.254) (layer "B.Cu") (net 12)))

